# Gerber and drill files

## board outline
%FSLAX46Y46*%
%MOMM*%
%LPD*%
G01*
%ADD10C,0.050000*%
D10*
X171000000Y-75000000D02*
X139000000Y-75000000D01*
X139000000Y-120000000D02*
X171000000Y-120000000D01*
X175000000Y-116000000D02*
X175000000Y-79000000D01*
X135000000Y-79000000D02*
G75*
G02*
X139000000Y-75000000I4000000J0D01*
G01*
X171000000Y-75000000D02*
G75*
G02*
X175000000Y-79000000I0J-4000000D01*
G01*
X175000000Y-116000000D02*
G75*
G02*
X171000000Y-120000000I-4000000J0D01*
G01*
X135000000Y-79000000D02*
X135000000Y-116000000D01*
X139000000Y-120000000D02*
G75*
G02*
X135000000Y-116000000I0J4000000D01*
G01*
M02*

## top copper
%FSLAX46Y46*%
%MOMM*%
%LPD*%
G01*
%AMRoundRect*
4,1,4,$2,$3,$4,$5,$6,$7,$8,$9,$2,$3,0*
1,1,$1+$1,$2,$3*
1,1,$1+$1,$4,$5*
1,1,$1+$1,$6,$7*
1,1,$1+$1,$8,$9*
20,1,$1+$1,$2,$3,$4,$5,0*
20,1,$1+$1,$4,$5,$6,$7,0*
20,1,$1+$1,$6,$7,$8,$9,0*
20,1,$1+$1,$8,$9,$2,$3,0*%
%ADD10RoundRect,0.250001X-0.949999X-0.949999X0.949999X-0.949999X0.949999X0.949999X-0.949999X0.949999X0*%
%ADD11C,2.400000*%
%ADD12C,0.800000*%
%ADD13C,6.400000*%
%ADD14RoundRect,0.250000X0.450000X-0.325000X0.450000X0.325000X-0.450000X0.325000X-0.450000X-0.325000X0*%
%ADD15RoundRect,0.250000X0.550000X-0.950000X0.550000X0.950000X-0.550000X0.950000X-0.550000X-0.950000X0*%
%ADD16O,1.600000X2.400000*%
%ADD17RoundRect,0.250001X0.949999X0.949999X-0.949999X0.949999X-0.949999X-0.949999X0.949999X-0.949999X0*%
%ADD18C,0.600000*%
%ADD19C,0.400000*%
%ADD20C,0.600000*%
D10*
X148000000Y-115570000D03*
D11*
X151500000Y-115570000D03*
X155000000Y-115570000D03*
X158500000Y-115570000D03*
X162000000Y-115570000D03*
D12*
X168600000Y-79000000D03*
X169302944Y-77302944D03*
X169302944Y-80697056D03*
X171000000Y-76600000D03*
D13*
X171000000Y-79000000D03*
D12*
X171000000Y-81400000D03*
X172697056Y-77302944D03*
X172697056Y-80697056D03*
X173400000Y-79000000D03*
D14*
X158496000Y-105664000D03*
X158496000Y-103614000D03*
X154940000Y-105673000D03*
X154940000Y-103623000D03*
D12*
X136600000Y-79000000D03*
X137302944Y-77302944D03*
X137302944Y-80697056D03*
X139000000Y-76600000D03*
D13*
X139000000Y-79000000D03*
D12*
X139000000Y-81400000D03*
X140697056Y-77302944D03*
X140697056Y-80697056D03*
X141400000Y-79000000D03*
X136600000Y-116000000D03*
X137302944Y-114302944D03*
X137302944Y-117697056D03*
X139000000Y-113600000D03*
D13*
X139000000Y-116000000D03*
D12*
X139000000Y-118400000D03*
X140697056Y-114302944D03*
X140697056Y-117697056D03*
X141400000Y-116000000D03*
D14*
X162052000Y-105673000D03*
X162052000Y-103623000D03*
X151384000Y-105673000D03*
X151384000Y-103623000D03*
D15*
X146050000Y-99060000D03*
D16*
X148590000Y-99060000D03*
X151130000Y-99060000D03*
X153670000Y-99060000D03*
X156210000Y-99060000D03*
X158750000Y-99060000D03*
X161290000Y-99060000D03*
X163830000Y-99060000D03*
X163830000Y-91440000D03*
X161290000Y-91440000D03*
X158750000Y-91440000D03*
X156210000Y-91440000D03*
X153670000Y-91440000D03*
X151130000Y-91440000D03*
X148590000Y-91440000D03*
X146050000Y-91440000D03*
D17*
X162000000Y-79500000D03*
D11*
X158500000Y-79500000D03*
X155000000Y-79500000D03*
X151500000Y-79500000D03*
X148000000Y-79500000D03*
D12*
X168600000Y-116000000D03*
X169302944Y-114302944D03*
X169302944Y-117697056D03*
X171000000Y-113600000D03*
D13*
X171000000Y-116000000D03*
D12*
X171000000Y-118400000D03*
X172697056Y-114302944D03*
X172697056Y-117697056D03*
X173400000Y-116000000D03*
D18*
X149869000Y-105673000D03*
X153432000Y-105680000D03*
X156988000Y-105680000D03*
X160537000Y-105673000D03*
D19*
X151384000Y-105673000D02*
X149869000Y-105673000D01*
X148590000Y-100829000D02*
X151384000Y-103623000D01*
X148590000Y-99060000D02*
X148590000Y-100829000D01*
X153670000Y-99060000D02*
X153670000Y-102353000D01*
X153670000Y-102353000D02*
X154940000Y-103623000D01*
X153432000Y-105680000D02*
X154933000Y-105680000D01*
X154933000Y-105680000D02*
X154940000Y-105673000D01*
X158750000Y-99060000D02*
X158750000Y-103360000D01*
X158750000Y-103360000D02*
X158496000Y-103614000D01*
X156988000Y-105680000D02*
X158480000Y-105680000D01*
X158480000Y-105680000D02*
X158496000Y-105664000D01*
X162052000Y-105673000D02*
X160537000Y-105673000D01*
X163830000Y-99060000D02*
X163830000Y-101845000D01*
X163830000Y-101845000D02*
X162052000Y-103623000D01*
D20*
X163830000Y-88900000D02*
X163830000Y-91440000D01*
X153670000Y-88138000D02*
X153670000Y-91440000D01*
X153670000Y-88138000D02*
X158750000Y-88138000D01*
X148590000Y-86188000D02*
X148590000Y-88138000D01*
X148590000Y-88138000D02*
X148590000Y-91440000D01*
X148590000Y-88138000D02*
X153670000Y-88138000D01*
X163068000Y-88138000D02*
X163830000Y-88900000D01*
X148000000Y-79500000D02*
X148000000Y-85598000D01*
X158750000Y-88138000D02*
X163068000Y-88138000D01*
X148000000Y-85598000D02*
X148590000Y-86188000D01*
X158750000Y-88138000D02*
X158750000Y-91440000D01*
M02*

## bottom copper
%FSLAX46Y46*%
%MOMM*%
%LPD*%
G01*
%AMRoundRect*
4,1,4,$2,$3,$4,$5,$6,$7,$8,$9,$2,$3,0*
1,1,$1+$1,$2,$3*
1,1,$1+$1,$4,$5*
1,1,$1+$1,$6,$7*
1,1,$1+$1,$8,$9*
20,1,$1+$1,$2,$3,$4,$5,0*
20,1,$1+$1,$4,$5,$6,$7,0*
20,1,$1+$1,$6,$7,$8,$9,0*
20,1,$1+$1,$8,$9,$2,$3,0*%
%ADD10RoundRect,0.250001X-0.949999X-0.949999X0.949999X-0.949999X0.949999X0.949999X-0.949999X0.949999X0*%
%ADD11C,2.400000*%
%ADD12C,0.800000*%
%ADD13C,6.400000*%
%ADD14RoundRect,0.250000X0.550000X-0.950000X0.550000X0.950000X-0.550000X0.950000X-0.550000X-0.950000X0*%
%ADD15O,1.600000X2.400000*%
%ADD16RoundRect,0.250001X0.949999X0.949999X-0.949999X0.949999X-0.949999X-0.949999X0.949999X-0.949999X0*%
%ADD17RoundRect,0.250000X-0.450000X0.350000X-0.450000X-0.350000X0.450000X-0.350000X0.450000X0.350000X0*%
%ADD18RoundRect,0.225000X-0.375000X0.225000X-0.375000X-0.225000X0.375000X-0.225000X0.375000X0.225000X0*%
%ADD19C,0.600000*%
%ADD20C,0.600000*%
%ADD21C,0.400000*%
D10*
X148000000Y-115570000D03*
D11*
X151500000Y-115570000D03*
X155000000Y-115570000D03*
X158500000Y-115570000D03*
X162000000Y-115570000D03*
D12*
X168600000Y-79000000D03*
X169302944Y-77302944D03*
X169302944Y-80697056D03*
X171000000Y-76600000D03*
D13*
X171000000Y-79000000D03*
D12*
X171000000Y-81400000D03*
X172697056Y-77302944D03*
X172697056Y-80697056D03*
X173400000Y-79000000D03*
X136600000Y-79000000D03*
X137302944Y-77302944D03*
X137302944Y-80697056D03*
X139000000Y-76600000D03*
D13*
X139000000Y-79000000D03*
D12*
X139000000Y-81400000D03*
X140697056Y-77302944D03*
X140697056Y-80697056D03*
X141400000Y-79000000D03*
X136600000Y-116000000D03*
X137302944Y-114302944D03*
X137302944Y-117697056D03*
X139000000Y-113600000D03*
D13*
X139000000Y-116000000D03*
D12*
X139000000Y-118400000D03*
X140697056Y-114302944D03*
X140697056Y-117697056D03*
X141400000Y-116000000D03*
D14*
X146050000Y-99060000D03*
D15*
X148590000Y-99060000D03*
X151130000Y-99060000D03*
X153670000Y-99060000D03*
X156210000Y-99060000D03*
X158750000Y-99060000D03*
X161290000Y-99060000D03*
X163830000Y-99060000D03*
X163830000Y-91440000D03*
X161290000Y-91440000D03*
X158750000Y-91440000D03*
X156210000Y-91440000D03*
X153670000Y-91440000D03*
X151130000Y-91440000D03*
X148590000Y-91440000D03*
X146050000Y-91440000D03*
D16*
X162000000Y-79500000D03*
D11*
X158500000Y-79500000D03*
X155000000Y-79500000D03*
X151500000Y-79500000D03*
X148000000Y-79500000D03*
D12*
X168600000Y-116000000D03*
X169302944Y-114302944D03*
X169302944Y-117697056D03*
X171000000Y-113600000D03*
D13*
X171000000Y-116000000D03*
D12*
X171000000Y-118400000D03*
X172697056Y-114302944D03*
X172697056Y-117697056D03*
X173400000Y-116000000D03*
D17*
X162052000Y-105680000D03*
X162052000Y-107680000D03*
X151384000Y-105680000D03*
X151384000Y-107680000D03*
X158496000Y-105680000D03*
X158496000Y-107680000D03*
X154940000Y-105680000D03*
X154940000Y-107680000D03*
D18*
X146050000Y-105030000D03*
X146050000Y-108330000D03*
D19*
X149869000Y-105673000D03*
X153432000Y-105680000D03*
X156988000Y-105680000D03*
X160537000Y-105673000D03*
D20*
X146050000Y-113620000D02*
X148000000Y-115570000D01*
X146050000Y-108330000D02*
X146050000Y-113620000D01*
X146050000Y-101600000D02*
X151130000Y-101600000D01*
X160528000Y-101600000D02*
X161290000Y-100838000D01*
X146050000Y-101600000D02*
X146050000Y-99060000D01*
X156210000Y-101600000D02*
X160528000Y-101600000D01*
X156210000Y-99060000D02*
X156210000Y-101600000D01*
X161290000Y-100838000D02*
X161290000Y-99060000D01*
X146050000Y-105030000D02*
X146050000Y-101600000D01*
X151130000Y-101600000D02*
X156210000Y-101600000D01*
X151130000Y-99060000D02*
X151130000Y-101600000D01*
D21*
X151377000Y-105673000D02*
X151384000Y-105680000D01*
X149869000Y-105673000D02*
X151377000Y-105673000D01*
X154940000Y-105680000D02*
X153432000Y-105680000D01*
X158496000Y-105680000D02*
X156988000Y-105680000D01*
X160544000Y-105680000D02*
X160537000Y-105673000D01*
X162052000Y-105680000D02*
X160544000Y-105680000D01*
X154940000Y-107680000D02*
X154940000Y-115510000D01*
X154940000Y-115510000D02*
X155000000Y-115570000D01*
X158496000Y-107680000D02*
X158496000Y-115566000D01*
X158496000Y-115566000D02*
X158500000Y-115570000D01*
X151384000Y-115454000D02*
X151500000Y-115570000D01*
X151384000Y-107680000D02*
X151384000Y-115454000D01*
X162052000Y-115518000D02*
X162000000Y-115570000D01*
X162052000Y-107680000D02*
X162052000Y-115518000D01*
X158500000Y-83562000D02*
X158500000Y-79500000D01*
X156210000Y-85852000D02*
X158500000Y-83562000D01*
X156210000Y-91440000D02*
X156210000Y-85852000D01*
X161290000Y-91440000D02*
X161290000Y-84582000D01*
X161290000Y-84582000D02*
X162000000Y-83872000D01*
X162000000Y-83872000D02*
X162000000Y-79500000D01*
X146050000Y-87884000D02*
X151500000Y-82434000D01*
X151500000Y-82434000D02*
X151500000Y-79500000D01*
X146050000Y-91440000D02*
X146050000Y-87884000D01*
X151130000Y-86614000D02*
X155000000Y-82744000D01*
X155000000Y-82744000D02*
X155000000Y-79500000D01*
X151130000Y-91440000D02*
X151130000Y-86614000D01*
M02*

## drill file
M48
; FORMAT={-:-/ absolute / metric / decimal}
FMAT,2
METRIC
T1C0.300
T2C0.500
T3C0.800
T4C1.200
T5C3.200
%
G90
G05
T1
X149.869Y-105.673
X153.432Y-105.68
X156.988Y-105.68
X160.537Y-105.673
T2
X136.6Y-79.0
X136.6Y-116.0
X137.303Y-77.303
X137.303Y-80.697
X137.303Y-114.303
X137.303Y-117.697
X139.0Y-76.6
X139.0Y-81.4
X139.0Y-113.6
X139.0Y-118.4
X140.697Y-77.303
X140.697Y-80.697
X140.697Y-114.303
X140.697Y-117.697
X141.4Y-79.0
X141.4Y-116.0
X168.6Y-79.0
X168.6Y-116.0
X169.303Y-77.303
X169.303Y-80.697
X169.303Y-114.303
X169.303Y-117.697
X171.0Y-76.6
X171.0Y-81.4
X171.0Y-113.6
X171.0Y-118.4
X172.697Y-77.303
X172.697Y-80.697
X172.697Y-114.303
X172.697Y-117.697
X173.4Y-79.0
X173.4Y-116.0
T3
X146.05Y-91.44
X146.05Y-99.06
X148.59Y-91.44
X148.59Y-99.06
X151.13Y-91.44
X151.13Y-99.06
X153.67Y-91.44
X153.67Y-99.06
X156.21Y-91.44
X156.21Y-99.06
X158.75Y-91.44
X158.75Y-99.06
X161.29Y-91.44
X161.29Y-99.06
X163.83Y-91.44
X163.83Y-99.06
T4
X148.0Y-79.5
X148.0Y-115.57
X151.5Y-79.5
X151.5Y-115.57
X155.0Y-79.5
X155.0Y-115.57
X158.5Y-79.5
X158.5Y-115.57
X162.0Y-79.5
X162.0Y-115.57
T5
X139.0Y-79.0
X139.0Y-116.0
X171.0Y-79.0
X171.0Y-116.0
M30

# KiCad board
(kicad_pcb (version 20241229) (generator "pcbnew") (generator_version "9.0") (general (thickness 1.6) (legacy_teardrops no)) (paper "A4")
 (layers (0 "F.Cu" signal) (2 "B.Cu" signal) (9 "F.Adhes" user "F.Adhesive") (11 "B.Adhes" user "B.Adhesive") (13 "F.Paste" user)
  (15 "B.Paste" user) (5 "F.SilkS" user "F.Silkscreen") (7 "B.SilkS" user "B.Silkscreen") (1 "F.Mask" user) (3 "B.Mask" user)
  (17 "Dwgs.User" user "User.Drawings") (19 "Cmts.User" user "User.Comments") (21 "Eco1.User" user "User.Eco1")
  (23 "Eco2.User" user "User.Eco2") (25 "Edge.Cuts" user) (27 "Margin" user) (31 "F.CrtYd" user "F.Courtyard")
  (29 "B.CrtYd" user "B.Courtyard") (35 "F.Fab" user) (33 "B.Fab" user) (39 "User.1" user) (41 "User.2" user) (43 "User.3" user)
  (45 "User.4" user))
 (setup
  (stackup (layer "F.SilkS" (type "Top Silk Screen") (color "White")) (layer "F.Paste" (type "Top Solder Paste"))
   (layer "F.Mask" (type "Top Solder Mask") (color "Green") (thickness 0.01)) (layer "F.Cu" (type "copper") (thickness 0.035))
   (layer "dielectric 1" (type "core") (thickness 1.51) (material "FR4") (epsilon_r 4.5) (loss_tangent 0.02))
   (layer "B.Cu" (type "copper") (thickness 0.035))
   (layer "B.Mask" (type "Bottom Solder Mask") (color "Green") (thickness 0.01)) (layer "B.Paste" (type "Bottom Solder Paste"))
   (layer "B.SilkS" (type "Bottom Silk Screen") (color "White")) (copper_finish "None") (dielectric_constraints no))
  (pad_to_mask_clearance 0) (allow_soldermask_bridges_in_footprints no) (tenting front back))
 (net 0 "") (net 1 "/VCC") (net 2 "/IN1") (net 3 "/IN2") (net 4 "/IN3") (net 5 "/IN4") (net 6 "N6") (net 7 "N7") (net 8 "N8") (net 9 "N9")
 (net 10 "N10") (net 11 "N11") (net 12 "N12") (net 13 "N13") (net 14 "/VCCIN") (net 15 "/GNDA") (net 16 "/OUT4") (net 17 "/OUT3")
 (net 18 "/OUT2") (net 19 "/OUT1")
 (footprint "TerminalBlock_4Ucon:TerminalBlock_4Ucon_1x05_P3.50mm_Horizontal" (layer "F.Cu") (at 148 115.57)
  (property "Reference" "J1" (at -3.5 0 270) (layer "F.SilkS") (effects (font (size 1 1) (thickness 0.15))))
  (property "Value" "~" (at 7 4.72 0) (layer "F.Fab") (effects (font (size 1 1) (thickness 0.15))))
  (pad "1" thru_hole roundrect (at 0 0) (size 2.4 2.4) (drill 1.2) (layers "*.Cu" "*.Mask") (remove_unused_layers no)
   (roundrect_rratio 0.104167) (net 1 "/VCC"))
  (pad "2" thru_hole circle (at 3.5 0) (size 2.4 2.4) (drill 1.2) (layers "*.Cu" "*.Mask") (remove_unused_layers no) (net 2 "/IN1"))
  (pad "3" thru_hole circle (at 7 0) (size 2.4 2.4) (drill 1.2) (layers "*.Cu" "*.Mask") (remove_unused_layers no) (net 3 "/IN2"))
  (pad "4" thru_hole circle (at 10.5 0) (size 2.4 2.4) (drill 1.2) (layers "*.Cu" "*.Mask") (remove_unused_layers no) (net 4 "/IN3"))
  (pad "5" thru_hole circle (at 14 0) (size 2.4 2.4) (drill 1.2) (layers "*.Cu" "*.Mask") (remove_unused_layers no) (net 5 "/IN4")))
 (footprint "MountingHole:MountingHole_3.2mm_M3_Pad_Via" (layer "F.Cu") (at 171 79)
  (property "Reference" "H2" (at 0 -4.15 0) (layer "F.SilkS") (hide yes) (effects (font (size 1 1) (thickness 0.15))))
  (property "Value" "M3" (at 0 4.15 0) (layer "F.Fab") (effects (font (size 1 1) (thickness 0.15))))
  (pad "1" thru_hole circle (at -2.4 0) (size 0.8 0.8) (drill 0.5) (layers "*.Cu" "*.Mask") (remove_unused_layers no) (zone_connect 2))
  (pad "1" thru_hole circle (at -1.697056 -1.697056) (size 0.8 0.8) (drill 0.5) (layers "*.Cu" "*.Mask") (remove_unused_layers no)
   (zone_connect 2))
  (pad "1" thru_hole circle (at -1.697056 1.697056) (size 0.8 0.8) (drill 0.5) (layers "*.Cu" "*.Mask") (remove_unused_layers no)
   (zone_connect 2))
  (pad "1" thru_hole circle (at 0 -2.4) (size 0.8 0.8) (drill 0.5) (layers "*.Cu" "*.Mask") (remove_unused_layers no) (zone_connect 2))
  (pad "1" thru_hole circle (at 0 0) (size 6.4 6.4) (drill 3.2) (layers "*.Cu" "*.Mask") (remove_unused_layers no) (zone_connect 2))
  (pad "1" thru_hole circle (at 0 2.4) (size 0.8 0.8) (drill 0.5) (layers "*.Cu" "*.Mask") (remove_unused_layers no) (zone_connect 2))
  (pad "1" thru_hole circle (at 1.697056 -1.697056) (size 0.8 0.8) (drill 0.5) (layers "*.Cu" "*.Mask") (remove_unused_layers no)
   (zone_connect 2))
  (pad "1" thru_hole circle (at 1.697056 1.697056) (size 0.8 0.8) (drill 0.5) (layers "*.Cu" "*.Mask") (remove_unused_layers no)
   (zone_connect 2))
  (pad "1" thru_hole circle (at 2.4 0) (size 0.8 0.8) (drill 0.5) (layers "*.Cu" "*.Mask") (remove_unused_layers no) (zone_connect 2)))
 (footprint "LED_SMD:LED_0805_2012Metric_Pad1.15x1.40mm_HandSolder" (layer "F.Cu") (at 158.496 104.639 90)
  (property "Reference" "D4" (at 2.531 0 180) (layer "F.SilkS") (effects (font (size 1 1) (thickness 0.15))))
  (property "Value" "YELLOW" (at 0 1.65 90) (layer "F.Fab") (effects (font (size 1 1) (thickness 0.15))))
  (pad "1" smd roundrect (at -1.025 0 90) (size 1.15 1.4) (layers "F.Cu" "F.Mask" "F.Paste") (roundrect_rratio 0.217391) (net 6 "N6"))
  (pad "2" smd roundrect (at 1.025 0 90) (size 1.15 1.4) (layers "F.Cu" "F.Mask" "F.Paste") (roundrect_rratio 0.217391) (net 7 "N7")))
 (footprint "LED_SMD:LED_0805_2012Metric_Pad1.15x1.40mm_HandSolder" (layer "F.Cu") (at 154.94 104.648 90)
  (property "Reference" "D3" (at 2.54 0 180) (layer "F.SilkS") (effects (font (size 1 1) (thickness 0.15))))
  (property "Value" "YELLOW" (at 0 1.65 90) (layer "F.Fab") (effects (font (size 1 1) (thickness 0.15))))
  (pad "1" smd roundrect (at -1.025 0 90) (size 1.15 1.4) (layers "F.Cu" "F.Mask" "F.Paste") (roundrect_rratio 0.217391) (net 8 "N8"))
  (pad "2" smd roundrect (at 1.025 0 90) (size 1.15 1.4) (layers "F.Cu" "F.Mask" "F.Paste") (roundrect_rratio 0.217391) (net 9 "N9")))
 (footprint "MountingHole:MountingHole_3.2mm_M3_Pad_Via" (layer "F.Cu") (at 139 79)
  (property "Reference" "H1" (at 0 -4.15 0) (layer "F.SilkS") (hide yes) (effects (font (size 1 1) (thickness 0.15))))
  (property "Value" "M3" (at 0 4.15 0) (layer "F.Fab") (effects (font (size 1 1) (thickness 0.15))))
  (pad "1" thru_hole circle (at -2.4 0) (size 0.8 0.8) (drill 0.5) (layers "*.Cu" "*.Mask") (remove_unused_layers no) (zone_connect 2))
  (pad "1" thru_hole circle (at -1.697056 -1.697056) (size 0.8 0.8) (drill 0.5) (layers "*.Cu" "*.Mask") (remove_unused_layers no)
   (zone_connect 2))
  (pad "1" thru_hole circle (at -1.697056 1.697056) (size 0.8 0.8) (drill 0.5) (layers "*.Cu" "*.Mask") (remove_unused_layers no)
   (zone_connect 2))
  (pad "1" thru_hole circle (at 0 -2.4) (size 0.8 0.8) (drill 0.5) (layers "*.Cu" "*.Mask") (remove_unused_layers no) (zone_connect 2))
  (pad "1" thru_hole circle (at 0 0) (size 6.4 6.4) (drill 3.2) (layers "*.Cu" "*.Mask") (remove_unused_layers no) (zone_connect 2))
  (pad "1" thru_hole circle (at 0 2.4) (size 0.8 0.8) (drill 0.5) (layers "*.Cu" "*.Mask") (remove_unused_layers no) (zone_connect 2))
  (pad "1" thru_hole circle (at 1.697056 -1.697056) (size 0.8 0.8) (drill 0.5) (layers "*.Cu" "*.Mask") (remove_unused_layers no)
   (zone_connect 2))
  (pad "1" thru_hole circle (at 1.697056 1.697056) (size 0.8 0.8) (drill 0.5) (layers "*.Cu" "*.Mask") (remove_unused_layers no)
   (zone_connect 2))
  (pad "1" thru_hole circle (at 2.4 0) (size 0.8 0.8) (drill 0.5) (layers "*.Cu" "*.Mask") (remove_unused_layers no) (zone_connect 2)))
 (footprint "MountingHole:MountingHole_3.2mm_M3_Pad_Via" (layer "F.Cu") (at 139 116)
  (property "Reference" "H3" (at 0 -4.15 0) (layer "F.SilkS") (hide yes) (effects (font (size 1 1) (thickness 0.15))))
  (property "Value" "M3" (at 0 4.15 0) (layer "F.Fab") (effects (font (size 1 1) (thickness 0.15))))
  (pad "1" thru_hole circle (at -2.4 0) (size 0.8 0.8) (drill 0.5) (layers "*.Cu" "*.Mask") (remove_unused_layers no) (zone_connect 2))
  (pad "1" thru_hole circle (at -1.697056 -1.697056) (size 0.8 0.8) (drill 0.5) (layers "*.Cu" "*.Mask") (remove_unused_layers no)
   (zone_connect 2))
  (pad "1" thru_hole circle (at -1.697056 1.697056) (size 0.8 0.8) (drill 0.5) (layers "*.Cu" "*.Mask") (remove_unused_layers no)
   (zone_connect 2))
  (pad "1" thru_hole circle (at 0 -2.4) (size 0.8 0.8) (drill 0.5) (layers "*.Cu" "*.Mask") (remove_unused_layers no) (zone_connect 2))
  (pad "1" thru_hole circle (at 0 0) (size 6.4 6.4) (drill 3.2) (layers "*.Cu" "*.Mask") (remove_unused_layers no) (zone_connect 2))
  (pad "1" thru_hole circle (at 0 2.4) (size 0.8 0.8) (drill 0.5) (layers "*.Cu" "*.Mask") (remove_unused_layers no) (zone_connect 2))
  (pad "1" thru_hole circle (at 1.697056 -1.697056) (size 0.8 0.8) (drill 0.5) (layers "*.Cu" "*.Mask") (remove_unused_layers no)
   (zone_connect 2))
  (pad "1" thru_hole circle (at 1.697056 1.697056) (size 0.8 0.8) (drill 0.5) (layers "*.Cu" "*.Mask") (remove_unused_layers no)
   (zone_connect 2))
  (pad "1" thru_hole circle (at 2.4 0) (size 0.8 0.8) (drill 0.5) (layers "*.Cu" "*.Mask") (remove_unused_layers no) (zone_connect 2)))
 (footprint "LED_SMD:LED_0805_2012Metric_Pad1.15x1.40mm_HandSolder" (layer "F.Cu") (at 162.052 104.648 90)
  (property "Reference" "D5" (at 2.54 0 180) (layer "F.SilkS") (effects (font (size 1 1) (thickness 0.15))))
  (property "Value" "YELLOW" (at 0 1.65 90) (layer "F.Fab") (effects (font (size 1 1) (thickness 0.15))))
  (pad "1" smd roundrect (at -1.025 0 90) (size 1.15 1.4) (layers "F.Cu" "F.Mask" "F.Paste") (roundrect_rratio 0.217391) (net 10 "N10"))
  (pad "2" smd roundrect (at 1.025 0 90) (size 1.15 1.4) (layers "F.Cu" "F.Mask" "F.Paste") (roundrect_rratio 0.217391) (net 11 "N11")))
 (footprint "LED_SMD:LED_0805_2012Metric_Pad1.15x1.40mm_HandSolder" (layer "F.Cu") (at 151.384 104.648 90)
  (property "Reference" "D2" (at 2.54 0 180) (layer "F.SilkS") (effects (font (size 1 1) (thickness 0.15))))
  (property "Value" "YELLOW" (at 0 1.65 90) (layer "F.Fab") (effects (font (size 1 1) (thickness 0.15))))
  (pad "1" smd roundrect (at -1.025 0 90) (size 1.15 1.4) (layers "F.Cu" "F.Mask" "F.Paste") (roundrect_rratio 0.217391) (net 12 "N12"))
  (pad "2" smd roundrect (at 1.025 0 90) (size 1.15 1.4) (layers "F.Cu" "F.Mask" "F.Paste") (roundrect_rratio 0.217391) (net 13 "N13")))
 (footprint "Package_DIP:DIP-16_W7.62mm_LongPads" (layer "F.Cu") (at 146.05 99.06 90)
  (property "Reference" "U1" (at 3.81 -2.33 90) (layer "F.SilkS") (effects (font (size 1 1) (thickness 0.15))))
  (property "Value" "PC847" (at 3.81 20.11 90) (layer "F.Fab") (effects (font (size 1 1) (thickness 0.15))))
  (pad "1" thru_hole roundrect (at 0 0 90) (size 2.4 1.6) (drill 0.8) (layers "*.Cu" "*.Mask") (remove_unused_layers no)
   (roundrect_rratio 0.15625) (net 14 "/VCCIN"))
  (pad "2" thru_hole oval (at 0 2.54 90) (size 2.4 1.6) (drill 0.8) (layers "*.Cu" "*.Mask") (remove_unused_layers no) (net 13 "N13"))
  (pad "3" thru_hole oval (at 0 5.08 90) (size 2.4 1.6) (drill 0.8) (layers "*.Cu" "*.Mask") (remove_unused_layers no) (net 14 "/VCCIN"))
  (pad "4" thru_hole oval (at 0 7.62 90) (size 2.4 1.6) (drill 0.8) (layers "*.Cu" "*.Mask") (remove_unused_layers no) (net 9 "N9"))
  (pad "5" thru_hole oval (at 0 10.16 90) (size 2.4 1.6) (drill 0.8) (layers "*.Cu" "*.Mask") (remove_unused_layers no) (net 14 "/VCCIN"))
  (pad "6" thru_hole oval (at 0 12.7 90) (size 2.4 1.6) (drill 0.8) (layers "*.Cu" "*.Mask") (remove_unused_layers no) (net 7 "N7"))
  (pad "7" thru_hole oval (at 0 15.24 90) (size 2.4 1.6) (drill 0.8) (layers "*.Cu" "*.Mask") (remove_unused_layers no) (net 14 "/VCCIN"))
  (pad "8" thru_hole oval (at 0 17.78 90) (size 2.4 1.6) (drill 0.8) (layers "*.Cu" "*.Mask") (remove_unused_layers no) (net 11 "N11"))
  (pad "9" thru_hole oval (at 7.62 17.78 90) (size 2.4 1.6) (drill 0.8) (layers "*.Cu" "*.Mask") (remove_unused_layers no) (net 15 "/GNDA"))
  (pad "10" thru_hole oval (at 7.62 15.24 90) (size 2.4 1.6) (drill 0.8) (layers "*.Cu" "*.Mask") (remove_unused_layers no) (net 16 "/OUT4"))
  (pad "11" thru_hole oval (at 7.62 12.7 90) (size 2.4 1.6) (drill 0.8) (layers "*.Cu" "*.Mask") (remove_unused_layers no) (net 15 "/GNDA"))
  (pad "12" thru_hole oval (at 7.62 10.16 90) (size 2.4 1.6) (drill 0.8) (layers "*.Cu" "*.Mask") (remove_unused_layers no) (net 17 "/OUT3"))
  (pad "13" thru_hole oval (at 7.62 7.62 90) (size 2.4 1.6) (drill 0.8) (layers "*.Cu" "*.Mask") (remove_unused_layers no) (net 15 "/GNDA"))
  (pad "14" thru_hole oval (at 7.62 5.08 90) (size 2.4 1.6) (drill 0.8) (layers "*.Cu" "*.Mask") (remove_unused_layers no) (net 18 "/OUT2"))
  (pad "15" thru_hole oval (at 7.62 2.54 90) (size 2.4 1.6) (drill 0.8) (layers "*.Cu" "*.Mask") (remove_unused_layers no) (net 15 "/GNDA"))
  (pad "16" thru_hole oval (at 7.62 0 90) (size 2.4 1.6) (drill 0.8) (layers "*.Cu" "*.Mask") (remove_unused_layers no) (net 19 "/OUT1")))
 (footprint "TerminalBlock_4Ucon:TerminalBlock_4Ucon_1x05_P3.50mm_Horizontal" (layer "F.Cu") (at 162 79.5 180)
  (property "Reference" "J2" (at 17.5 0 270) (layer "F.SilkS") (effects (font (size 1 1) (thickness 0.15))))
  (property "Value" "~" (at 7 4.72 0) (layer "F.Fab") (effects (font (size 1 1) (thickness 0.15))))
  (pad "1" thru_hole roundrect (at 0 0 180) (size 2.4 2.4) (drill 1.2) (layers "*.Cu" "*.Mask") (remove_unused_layers no)
   (roundrect_rratio 0.104167) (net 16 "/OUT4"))
  (pad "2" thru_hole circle (at 3.5 0 180) (size 2.4 2.4) (drill 1.2) (layers "*.Cu" "*.Mask") (remove_unused_layers no) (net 17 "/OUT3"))
  (pad "3" thru_hole circle (at 7 0 180) (size 2.4 2.4) (drill 1.2) (layers "*.Cu" "*.Mask") (remove_unused_layers no) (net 18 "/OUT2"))
  (pad "4" thru_hole circle (at 10.5 0 180) (size 2.4 2.4) (drill 1.2) (layers "*.Cu" "*.Mask") (remove_unused_layers no) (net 19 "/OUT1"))
  (pad "5" thru_hole circle (at 14 0 180) (size 2.4 2.4) (drill 1.2) (layers "*.Cu" "*.Mask") (remove_unused_layers no) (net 15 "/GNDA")))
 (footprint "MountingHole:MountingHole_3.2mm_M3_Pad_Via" (layer "F.Cu") (at 171 116)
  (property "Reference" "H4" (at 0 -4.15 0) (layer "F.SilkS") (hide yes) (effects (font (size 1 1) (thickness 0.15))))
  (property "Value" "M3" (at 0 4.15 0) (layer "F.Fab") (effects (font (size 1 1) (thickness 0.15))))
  (pad "1" thru_hole circle (at -2.4 0) (size 0.8 0.8) (drill 0.5) (layers "*.Cu" "*.Mask") (remove_unused_layers no) (zone_connect 2))
  (pad "1" thru_hole circle (at -1.697056 -1.697056) (size 0.8 0.8) (drill 0.5) (layers "*.Cu" "*.Mask") (remove_unused_layers no)
   (zone_connect 2))
  (pad "1" thru_hole circle (at -1.697056 1.697056) (size 0.8 0.8) (drill 0.5) (layers "*.Cu" "*.Mask") (remove_unused_layers no)
   (zone_connect 2))
  (pad "1" thru_hole circle (at 0 -2.4) (size 0.8 0.8) (drill 0.5) (layers "*.Cu" "*.Mask") (remove_unused_layers no) (zone_connect 2))
  (pad "1" thru_hole circle (at 0 0) (size 6.4 6.4) (drill 3.2) (layers "*.Cu" "*.Mask") (remove_unused_layers no) (zone_connect 2))
  (pad "1" thru_hole circle (at 0 2.4) (size 0.8 0.8) (drill 0.5) (layers "*.Cu" "*.Mask") (remove_unused_layers no) (zone_connect 2))
  (pad "1" thru_hole circle (at 1.697056 -1.697056) (size 0.8 0.8) (drill 0.5) (layers "*.Cu" "*.Mask") (remove_unused_layers no)
   (zone_connect 2))
  (pad "1" thru_hole circle (at 1.697056 1.697056) (size 0.8 0.8) (drill 0.5) (layers "*.Cu" "*.Mask") (remove_unused_layers no)
   (zone_connect 2))
  (pad "1" thru_hole circle (at 2.4 0) (size 0.8 0.8) (drill 0.5) (layers "*.Cu" "*.Mask") (remove_unused_layers no) (zone_connect 2)))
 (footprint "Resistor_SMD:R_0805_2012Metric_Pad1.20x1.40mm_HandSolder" (layer "B.Cu") (at 162.052 106.68 -90)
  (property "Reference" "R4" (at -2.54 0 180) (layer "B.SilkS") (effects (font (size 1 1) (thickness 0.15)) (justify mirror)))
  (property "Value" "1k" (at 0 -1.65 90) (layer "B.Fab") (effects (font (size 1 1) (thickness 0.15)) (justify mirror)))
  (pad "1" smd roundrect (at -1 0 270) (size 1.2 1.4) (layers "B.Cu" "B.Mask" "B.Paste") (roundrect_rratio 0.208333) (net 10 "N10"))
  (pad "2" smd roundrect (at 1 0 270) (size 1.2 1.4) (layers "B.Cu" "B.Mask" "B.Paste") (roundrect_rratio 0.208333) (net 5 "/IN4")))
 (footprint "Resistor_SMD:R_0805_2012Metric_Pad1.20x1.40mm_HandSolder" (layer "B.Cu") (at 151.384 106.68 -90)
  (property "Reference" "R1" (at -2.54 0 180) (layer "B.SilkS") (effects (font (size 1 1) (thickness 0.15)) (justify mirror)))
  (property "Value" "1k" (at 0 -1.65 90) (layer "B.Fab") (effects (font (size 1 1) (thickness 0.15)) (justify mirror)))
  (pad "1" smd roundrect (at -1 0 270) (size 1.2 1.4) (layers "B.Cu" "B.Mask" "B.Paste") (roundrect_rratio 0.208333) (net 12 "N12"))
  (pad "2" smd roundrect (at 1 0 270) (size 1.2 1.4) (layers "B.Cu" "B.Mask" "B.Paste") (roundrect_rratio 0.208333) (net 2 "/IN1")))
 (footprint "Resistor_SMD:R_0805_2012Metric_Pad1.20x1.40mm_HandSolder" (layer "B.Cu") (at 158.496 106.68 -90)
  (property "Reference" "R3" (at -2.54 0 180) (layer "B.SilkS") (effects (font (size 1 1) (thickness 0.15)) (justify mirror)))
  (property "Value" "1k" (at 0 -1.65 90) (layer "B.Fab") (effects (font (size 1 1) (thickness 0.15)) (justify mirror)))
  (pad "1" smd roundrect (at -1 0 270) (size 1.2 1.4) (layers "B.Cu" "B.Mask" "B.Paste") (roundrect_rratio 0.208333) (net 6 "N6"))
  (pad "2" smd roundrect (at 1 0 270) (size 1.2 1.4) (layers "B.Cu" "B.Mask" "B.Paste") (roundrect_rratio 0.208333) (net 4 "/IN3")))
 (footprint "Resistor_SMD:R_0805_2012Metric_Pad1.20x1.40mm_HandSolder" (layer "B.Cu") (at 154.94 106.68 -90)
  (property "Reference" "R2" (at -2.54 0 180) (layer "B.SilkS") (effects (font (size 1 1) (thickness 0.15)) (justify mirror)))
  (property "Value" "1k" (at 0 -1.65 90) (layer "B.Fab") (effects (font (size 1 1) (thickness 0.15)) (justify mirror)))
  (pad "1" smd roundrect (at -1 0 270) (size 1.2 1.4) (layers "B.Cu" "B.Mask" "B.Paste") (roundrect_rratio 0.208333) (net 8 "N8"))
  (pad "2" smd roundrect (at 1 0 270) (size 1.2 1.4) (layers "B.Cu" "B.Mask" "B.Paste") (roundrect_rratio 0.208333) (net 3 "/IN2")))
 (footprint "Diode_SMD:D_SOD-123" (layer "B.Cu") (at 146.05 106.68 -90)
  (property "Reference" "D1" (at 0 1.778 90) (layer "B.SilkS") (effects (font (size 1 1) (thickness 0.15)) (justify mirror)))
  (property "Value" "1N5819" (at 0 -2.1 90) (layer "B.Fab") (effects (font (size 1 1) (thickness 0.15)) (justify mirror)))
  (pad "1" smd roundrect (at -1.65 0 270) (size 0.9 1.2) (layers "B.Cu" "B.Mask" "B.Paste") (roundrect_rratio 0.25) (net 14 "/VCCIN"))
  (pad "2" smd roundrect (at 1.65 0 270) (size 0.9 1.2) (layers "B.Cu" "B.Mask" "B.Paste") (roundrect_rratio 0.25) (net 1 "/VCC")))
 (gr_line (start 171 75) (end 139 75) (stroke (width 0.05) (type default)) (layer "Edge.Cuts"))
 (gr_line (start 139 120) (end 171 120) (stroke (width 0.05) (type default)) (layer "Edge.Cuts"))
 (gr_line (start 175 116) (end 175 79) (stroke (width 0.05) (type default)) (layer "Edge.Cuts"))
 (gr_arc (start 135 79) (mid 136.171573 76.171573) (end 139 75) (stroke (width 0.05) (type default)) (layer "Edge.Cuts"))
 (gr_arc (start 171 75) (mid 173.828427 76.171573) (end 175 79) (stroke (width 0.05) (type default)) (layer "Edge.Cuts"))
 (gr_arc (start 175 116) (mid 173.828427 118.828427) (end 171 120) (stroke (width 0.05) (type default)) (layer "Edge.Cuts"))
 (gr_line (start 135 79) (end 135 116) (stroke (width 0.05) (type default)) (layer "Edge.Cuts"))
 (gr_arc (start 139 120) (mid 136.171573 118.828427) (end 135 116) (stroke (width 0.05) (type default)) (layer "Edge.Cuts"))
 (segment (start 146.05 113.62) (end 148 115.57) (width 0.6) (layer "B.Cu") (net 1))
 (segment (start 146.05 108.33) (end 146.05 113.62) (width 0.6) (layer "B.Cu") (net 1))
 (segment (start 146.05 101.6) (end 151.13 101.6) (width 0.6) (layer "B.Cu") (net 14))
 (segment (start 160.528 101.6) (end 161.29 100.838) (width 0.6) (layer "B.Cu") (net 14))
 (segment (start 146.05 101.6) (end 146.05 99.06) (width 0.6) (layer "B.Cu") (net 14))
 (segment (start 156.21 101.6) (end 160.528 101.6) (width 0.6) (layer "B.Cu") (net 14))
 (segment (start 156.21 99.06) (end 156.21 101.6) (width 0.6) (layer "B.Cu") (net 14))
 (segment (start 161.29 100.838) (end 161.29 99.06) (width 0.6) (layer "B.Cu") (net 14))
 (segment (start 146.05 105.03) (end 146.05 101.6) (width 0.6) (layer "B.Cu") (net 14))
 (segment (start 151.13 101.6) (end 156.21 101.6) (width 0.6) (layer "B.Cu") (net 14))
 (segment (start 151.13 99.06) (end 151.13 101.6) (width 0.6) (layer "B.Cu") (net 14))
 (segment (start 151.384 105.673) (end 149.869 105.673) (width 0.4) (layer "F.Cu") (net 12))
 (via (at 149.869 105.673) (size 0.6) (drill 0.3) (layers "F.Cu" "B.Cu") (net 12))
 (segment (start 151.377 105.673) (end 151.384 105.68) (width 0.4) (layer "B.Cu") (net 12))
 (segment (start 149.869 105.673) (end 151.377 105.673) (width 0.4) (layer "B.Cu") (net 12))
 (segment (start 148.59 100.829) (end 151.384 103.623) (width 0.4) (layer "F.Cu") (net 13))
 (segment (start 148.59 99.06) (end 148.59 100.829) (width 0.4) (layer "F.Cu") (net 13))
 (segment (start 153.67 99.06) (end 153.67 102.353) (width 0.4) (layer "F.Cu") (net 9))
 (segment (start 153.67 102.353) (end 154.94 103.623) (width 0.4) (layer "F.Cu") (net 9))
 (segment (start 153.432 105.68) (end 154.933 105.68) (width 0.4) (layer "F.Cu") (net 8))
 (segment (start 154.933 105.68) (end 154.94 105.673) (width 0.4) (layer "F.Cu") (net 8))
 (via (at 153.432 105.68) (size 0.6) (drill 0.3) (layers "F.Cu" "B.Cu") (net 8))
 (segment (start 154.94 105.68) (end 153.432 105.68) (width 0.4) (layer "B.Cu") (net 8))
 (segment (start 158.75 99.06) (end 158.75 103.36) (width 0.4) (layer "F.Cu") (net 7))
 (segment (start 158.75 103.36) (end 158.496 103.614) (width 0.4) (layer "F.Cu") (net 7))
 (segment (start 156.988 105.68) (end 158.48 105.68) (width 0.4) (layer "F.Cu") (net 6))
 (segment (start 158.48 105.68) (end 158.496 105.664) (width 0.4) (layer "F.Cu") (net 6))
 (via (at 156.988 105.68) (size 0.6) (drill 0.3) (layers "F.Cu" "B.Cu") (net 6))
 (segment (start 158.496 105.68) (end 156.988 105.68) (width 0.4) (layer "B.Cu") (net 6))
 (segment (start 162.052 105.673) (end 160.537 105.673) (width 0.4) (layer "F.Cu") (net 10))
 (via (at 160.537 105.673) (size 0.6) (drill 0.3) (layers "F.Cu" "B.Cu") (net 10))
 (segment (start 160.544 105.68) (end 160.537 105.673) (width 0.4) (layer "B.Cu") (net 10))
 (segment (start 162.052 105.68) (end 160.544 105.68) (width 0.4) (layer "B.Cu") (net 10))
 (segment (start 163.83 99.06) (end 163.83 101.845) (width 0.4) (layer "F.Cu") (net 11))
 (segment (start 163.83 101.845) (end 162.052 103.623) (width 0.4) (layer "F.Cu") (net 11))
 (segment (start 154.94 107.68) (end 154.94 115.51) (width 0.4) (layer "B.Cu") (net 3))
 (segment (start 154.94 115.51) (end 155 115.57) (width 0.4) (layer "B.Cu") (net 3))
 (segment (start 158.496 107.68) (end 158.496 115.566) (width 0.4) (layer "B.Cu") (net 4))
 (segment (start 158.496 115.566) (end 158.5 115.57) (width 0.4) (layer "B.Cu") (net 4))
 (segment (start 151.384 115.454) (end 151.5 115.57) (width 0.4) (layer "B.Cu") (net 2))
 (segment (start 151.384 107.68) (end 151.384 115.454) (width 0.4) (layer "B.Cu") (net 2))
 (segment (start 162.052 115.518) (end 162 115.57) (width 0.4) (layer "B.Cu") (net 5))
 (segment (start 162.052 107.68) (end 162.052 115.518) (width 0.4) (layer "B.Cu") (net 5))
 (segment (start 158.5 83.562) (end 158.5 79.5) (width 0.4) (layer "B.Cu") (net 17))
 (segment (start 156.21 85.852) (end 158.5 83.562) (width 0.4) (layer "B.Cu") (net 17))
 (segment (start 156.21 91.44) (end 156.21 85.852) (width 0.4) (layer "B.Cu") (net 17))
 (segment (start 163.83 88.9) (end 163.83 91.44) (width 0.6) (layer "F.Cu") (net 15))
 (segment (start 153.67 88.138) (end 153.67 91.44) (width 0.6) (layer "F.Cu") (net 15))
 (segment (start 153.67 88.138) (end 158.75 88.138) (width 0.6) (layer "F.Cu") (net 15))
 (segment (start 148.59 86.188) (end 148.59 88.138) (width 0.6) (layer "F.Cu") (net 15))
 (segment (start 148.59 88.138) (end 148.59 91.44) (width 0.6) (layer "F.Cu") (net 15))
 (segment (start 148.59 88.138) (end 153.67 88.138) (width 0.6) (layer "F.Cu") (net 15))
 (segment (start 163.068 88.138) (end 163.83 88.9) (width 0.6) (layer "F.Cu") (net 15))
 (segment (start 148 79.5) (end 148 85.598) (width 0.6) (layer "F.Cu") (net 15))
 (segment (start 158.75 88.138) (end 163.068 88.138) (width 0.6) (layer "F.Cu") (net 15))
 (segment (start 148 85.598) (end 148.59 86.188) (width 0.6) (layer "F.Cu") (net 15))
 (segment (start 158.75 88.138) (end 158.75 91.44) (width 0.6) (layer "F.Cu") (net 15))
 (segment (start 161.29 91.44) (end 161.29 84.582) (width 0.4) (layer "B.Cu") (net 16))
 (segment (start 161.29 84.582) (end 162 83.872) (width 0.4) (layer "B.Cu") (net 16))
 (segment (start 162 83.872) (end 162 79.5) (width 0.4) (layer "B.Cu") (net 16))
 (segment (start 146.05 87.884) (end 151.5 82.434) (width 0.4) (layer "B.Cu") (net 19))
 (segment (start 151.5 82.434) (end 151.5 79.5) (width 0.4) (layer "B.Cu") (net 19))
 (segment (start 146.05 91.44) (end 146.05 87.884) (width 0.4) (layer "B.Cu") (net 19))
 (segment (start 151.13 86.614) (end 155 82.744) (width 0.4) (layer "B.Cu") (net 18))
 (segment (start 155 82.744) (end 155 79.5) (width 0.4) (layer "B.Cu") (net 18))
 (segment (start 151.13 91.44) (end 151.13 86.614) (width 0.4) (layer "B.Cu") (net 18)))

